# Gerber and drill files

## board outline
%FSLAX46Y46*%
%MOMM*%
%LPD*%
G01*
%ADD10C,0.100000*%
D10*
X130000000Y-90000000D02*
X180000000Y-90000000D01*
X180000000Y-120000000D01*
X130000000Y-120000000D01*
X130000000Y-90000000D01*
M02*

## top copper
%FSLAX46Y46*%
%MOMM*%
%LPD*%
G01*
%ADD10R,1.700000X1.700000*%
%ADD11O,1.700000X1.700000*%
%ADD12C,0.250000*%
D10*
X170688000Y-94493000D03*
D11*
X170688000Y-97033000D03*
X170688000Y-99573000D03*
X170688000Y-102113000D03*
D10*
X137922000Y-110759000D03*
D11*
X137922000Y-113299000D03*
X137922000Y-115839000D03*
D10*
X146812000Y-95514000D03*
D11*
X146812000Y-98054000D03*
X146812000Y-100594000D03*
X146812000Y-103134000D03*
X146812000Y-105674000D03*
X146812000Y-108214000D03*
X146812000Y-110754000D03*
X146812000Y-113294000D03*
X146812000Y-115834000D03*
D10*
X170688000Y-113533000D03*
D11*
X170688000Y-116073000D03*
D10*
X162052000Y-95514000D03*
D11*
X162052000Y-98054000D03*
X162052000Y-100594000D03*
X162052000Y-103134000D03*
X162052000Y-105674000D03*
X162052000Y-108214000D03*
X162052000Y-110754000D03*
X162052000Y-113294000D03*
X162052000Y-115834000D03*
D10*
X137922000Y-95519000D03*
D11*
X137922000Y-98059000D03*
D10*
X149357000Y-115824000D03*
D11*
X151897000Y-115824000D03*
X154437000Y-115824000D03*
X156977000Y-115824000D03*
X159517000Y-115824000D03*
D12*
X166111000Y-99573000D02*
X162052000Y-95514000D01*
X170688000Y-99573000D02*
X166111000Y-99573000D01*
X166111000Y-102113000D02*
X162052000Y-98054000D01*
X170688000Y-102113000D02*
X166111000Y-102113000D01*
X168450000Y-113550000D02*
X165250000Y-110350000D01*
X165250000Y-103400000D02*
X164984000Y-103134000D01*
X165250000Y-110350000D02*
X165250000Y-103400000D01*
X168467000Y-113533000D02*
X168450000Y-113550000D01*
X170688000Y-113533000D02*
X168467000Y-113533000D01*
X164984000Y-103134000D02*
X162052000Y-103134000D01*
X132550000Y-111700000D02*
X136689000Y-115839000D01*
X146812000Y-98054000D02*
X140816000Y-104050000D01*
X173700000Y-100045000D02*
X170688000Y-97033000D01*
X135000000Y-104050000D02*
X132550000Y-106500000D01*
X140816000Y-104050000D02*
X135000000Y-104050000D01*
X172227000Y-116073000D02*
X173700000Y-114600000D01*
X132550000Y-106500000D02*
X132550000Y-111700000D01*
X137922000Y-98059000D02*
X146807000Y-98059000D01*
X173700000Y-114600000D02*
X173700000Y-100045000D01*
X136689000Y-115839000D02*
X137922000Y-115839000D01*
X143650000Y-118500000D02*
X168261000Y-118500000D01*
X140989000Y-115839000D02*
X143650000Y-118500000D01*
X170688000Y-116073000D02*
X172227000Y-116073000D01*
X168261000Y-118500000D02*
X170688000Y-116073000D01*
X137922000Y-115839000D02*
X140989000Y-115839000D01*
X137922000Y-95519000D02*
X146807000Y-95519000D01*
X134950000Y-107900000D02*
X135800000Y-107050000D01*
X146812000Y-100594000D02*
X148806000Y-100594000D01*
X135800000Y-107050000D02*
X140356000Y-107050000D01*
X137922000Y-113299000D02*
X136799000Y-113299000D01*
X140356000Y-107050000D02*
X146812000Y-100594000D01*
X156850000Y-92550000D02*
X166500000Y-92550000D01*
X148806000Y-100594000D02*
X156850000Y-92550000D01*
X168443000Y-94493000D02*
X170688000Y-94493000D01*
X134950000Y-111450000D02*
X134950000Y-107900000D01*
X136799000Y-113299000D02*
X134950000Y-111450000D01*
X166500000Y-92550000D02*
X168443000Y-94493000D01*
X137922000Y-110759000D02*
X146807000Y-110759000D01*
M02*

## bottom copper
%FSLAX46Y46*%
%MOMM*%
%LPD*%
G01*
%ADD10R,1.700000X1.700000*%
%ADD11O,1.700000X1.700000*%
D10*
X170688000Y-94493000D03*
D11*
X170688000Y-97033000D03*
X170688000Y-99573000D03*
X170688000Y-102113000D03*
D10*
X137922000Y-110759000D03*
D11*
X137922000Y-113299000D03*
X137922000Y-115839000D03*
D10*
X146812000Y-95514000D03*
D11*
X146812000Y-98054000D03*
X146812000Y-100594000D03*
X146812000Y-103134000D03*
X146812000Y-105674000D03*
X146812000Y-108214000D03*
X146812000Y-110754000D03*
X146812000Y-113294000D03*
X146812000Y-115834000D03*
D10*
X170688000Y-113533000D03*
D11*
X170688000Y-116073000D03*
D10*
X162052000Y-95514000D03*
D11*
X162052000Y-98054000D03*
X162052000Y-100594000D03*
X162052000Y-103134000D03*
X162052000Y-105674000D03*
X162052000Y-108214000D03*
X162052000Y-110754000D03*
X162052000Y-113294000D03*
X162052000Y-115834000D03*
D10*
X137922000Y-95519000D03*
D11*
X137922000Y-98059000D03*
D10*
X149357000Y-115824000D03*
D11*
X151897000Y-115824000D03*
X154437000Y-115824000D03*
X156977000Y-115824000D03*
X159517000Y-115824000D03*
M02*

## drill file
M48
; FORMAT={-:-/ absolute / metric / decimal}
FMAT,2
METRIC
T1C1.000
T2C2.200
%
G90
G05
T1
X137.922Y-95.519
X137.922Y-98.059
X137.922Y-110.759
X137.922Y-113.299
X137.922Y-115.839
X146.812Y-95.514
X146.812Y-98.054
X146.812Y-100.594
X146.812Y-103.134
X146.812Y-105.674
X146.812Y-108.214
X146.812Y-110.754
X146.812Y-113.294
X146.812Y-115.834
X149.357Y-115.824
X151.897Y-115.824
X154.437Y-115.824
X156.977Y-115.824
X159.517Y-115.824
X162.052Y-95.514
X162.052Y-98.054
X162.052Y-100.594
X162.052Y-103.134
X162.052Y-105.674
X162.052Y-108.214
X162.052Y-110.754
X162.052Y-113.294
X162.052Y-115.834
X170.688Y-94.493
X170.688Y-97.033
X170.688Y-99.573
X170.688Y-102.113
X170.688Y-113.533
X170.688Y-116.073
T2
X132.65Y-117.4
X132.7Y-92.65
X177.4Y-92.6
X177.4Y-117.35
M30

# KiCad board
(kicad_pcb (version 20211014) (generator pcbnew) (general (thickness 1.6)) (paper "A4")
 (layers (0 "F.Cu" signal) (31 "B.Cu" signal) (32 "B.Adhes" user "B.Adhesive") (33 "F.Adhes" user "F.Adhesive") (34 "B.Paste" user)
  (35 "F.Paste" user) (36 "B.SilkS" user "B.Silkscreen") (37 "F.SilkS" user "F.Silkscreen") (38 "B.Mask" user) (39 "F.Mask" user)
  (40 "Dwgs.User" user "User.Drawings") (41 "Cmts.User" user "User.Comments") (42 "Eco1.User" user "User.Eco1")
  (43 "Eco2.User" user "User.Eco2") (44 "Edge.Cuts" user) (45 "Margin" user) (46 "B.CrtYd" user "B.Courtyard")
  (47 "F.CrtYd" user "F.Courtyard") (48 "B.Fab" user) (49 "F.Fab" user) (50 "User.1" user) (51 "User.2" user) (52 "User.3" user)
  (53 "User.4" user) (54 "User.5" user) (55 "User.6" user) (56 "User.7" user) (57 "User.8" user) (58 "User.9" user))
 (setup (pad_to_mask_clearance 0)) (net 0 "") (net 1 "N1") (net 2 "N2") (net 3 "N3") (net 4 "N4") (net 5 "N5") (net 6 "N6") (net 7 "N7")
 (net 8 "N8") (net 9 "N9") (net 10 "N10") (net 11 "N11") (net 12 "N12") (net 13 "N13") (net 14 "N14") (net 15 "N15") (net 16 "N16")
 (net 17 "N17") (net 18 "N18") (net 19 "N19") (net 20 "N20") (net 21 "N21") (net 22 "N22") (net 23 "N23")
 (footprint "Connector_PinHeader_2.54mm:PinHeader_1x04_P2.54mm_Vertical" (layer "F.Cu") (at 170.688 94.493)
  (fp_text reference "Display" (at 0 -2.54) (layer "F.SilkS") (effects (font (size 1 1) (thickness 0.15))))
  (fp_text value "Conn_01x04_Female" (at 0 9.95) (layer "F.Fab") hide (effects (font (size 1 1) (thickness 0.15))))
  (pad "1" thru_hole rect (at 0 0) (size 1.7 1.7) (drill 1) (layers *.Cu *.Mask) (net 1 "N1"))
  (pad "2" thru_hole oval (at 0 2.54) (size 1.7 1.7) (drill 1) (layers *.Cu *.Mask) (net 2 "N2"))
  (pad "3" thru_hole oval (at 0 5.08) (size 1.7 1.7) (drill 1) (layers *.Cu *.Mask) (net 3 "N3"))
  (pad "4" thru_hole oval (at 0 7.62) (size 1.7 1.7) (drill 1) (layers *.Cu *.Mask) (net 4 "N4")))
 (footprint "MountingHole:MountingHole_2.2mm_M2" (layer "F.Cu") (at 177.4 92.6)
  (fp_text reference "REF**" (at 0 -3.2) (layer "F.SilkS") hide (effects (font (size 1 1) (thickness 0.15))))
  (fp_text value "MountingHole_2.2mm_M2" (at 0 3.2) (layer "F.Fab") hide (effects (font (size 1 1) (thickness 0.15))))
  (pad "" np_thru_hole circle (at 0 0) (size 2.2 2.2) (drill 2.2) (layers *.Cu *.Mask)))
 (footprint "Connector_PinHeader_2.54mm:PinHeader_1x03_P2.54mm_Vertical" (layer "F.Cu") (at 137.922 110.759)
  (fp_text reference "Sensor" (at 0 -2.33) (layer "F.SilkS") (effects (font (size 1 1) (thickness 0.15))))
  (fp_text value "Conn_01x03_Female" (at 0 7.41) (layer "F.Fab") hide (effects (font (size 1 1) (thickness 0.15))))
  (pad "1" thru_hole rect (at 0 0) (size 1.7 1.7) (drill 1) (layers *.Cu *.Mask) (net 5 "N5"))
  (pad "2" thru_hole oval (at 0 2.54) (size 1.7 1.7) (drill 1) (layers *.Cu *.Mask) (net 1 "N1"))
  (pad "3" thru_hole oval (at 0 5.08) (size 1.7 1.7) (drill 1) (layers *.Cu *.Mask) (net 2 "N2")))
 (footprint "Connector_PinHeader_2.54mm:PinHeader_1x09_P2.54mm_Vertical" (layer "F.Cu") (at 146.812 95.514)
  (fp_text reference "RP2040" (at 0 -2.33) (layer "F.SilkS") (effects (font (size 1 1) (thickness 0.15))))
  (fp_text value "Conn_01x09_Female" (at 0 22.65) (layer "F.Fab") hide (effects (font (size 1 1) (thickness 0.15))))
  (pad "1" thru_hole rect (at 0 0) (size 1.7 1.7) (drill 1) (layers *.Cu *.Mask) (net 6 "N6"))
  (pad "2" thru_hole oval (at 0 2.54) (size 1.7 1.7) (drill 1) (layers *.Cu *.Mask) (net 2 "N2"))
  (pad "3" thru_hole oval (at 0 5.08) (size 1.7 1.7) (drill 1) (layers *.Cu *.Mask) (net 1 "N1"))
  (pad "4" thru_hole oval (at 0 7.62) (size 1.7 1.7) (drill 1) (layers *.Cu *.Mask) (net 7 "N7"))
  (pad "5" thru_hole oval (at 0 10.16) (size 1.7 1.7) (drill 1) (layers *.Cu *.Mask) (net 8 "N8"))
  (pad "6" thru_hole oval (at 0 12.7) (size 1.7 1.7) (drill 1) (layers *.Cu *.Mask) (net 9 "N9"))
  (pad "7" thru_hole oval (at 0 15.24) (size 1.7 1.7) (drill 1) (layers *.Cu *.Mask) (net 5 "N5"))
  (pad "8" thru_hole oval (at 0 17.78) (size 1.7 1.7) (drill 1) (layers *.Cu *.Mask) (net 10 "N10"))
  (pad "9" thru_hole oval (at 0 20.32) (size 1.7 1.7) (drill 1) (layers *.Cu *.Mask) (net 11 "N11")))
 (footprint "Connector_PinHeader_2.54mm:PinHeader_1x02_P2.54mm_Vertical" (layer "F.Cu") (at 170.688 113.533)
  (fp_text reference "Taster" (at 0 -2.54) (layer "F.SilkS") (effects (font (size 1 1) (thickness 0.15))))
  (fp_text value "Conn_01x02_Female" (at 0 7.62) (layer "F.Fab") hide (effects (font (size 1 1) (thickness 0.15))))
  (pad "1" thru_hole rect (at 0 0) (size 1.7 1.7) (drill 1) (layers *.Cu *.Mask) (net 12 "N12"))
  (pad "2" thru_hole oval (at 0 2.54) (size 1.7 1.7) (drill 1) (layers *.Cu *.Mask) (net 2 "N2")))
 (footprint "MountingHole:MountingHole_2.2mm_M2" (layer "F.Cu") (at 132.7 92.65)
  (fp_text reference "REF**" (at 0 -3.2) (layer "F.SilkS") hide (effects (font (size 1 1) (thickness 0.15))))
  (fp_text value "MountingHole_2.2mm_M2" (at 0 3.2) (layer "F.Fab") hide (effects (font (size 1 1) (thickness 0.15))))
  (pad "" np_thru_hole circle (at 0 0) (size 2.2 2.2) (drill 2.2) (layers *.Cu *.Mask)))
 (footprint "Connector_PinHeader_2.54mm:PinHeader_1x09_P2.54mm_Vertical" (layer "F.Cu") (at 162.052 95.514)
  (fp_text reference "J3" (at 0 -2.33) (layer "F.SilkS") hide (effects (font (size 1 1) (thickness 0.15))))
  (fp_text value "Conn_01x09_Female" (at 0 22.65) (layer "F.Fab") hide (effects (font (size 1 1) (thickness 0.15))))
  (pad "1" thru_hole rect (at 0 0) (size 1.7 1.7) (drill 1) (layers *.Cu *.Mask) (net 3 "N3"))
  (pad "2" thru_hole oval (at 0 2.54) (size 1.7 1.7) (drill 1) (layers *.Cu *.Mask) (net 4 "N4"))
  (pad "3" thru_hole oval (at 0 5.08) (size 1.7 1.7) (drill 1) (layers *.Cu *.Mask) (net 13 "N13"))
  (pad "4" thru_hole oval (at 0 7.62) (size 1.7 1.7) (drill 1) (layers *.Cu *.Mask) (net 12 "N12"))
  (pad "5" thru_hole oval (at 0 10.16) (size 1.7 1.7) (drill 1) (layers *.Cu *.Mask) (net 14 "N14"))
  (pad "6" thru_hole oval (at 0 12.7) (size 1.7 1.7) (drill 1) (layers *.Cu *.Mask) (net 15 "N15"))
  (pad "7" thru_hole oval (at 0 15.24) (size 1.7 1.7) (drill 1) (layers *.Cu *.Mask) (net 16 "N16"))
  (pad "8" thru_hole oval (at 0 17.78) (size 1.7 1.7) (drill 1) (layers *.Cu *.Mask) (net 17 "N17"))
  (pad "9" thru_hole oval (at 0 20.32) (size 1.7 1.7) (drill 1) (layers *.Cu *.Mask) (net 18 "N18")))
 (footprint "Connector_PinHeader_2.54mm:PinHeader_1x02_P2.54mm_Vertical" (layer "F.Cu") (at 137.922 95.519)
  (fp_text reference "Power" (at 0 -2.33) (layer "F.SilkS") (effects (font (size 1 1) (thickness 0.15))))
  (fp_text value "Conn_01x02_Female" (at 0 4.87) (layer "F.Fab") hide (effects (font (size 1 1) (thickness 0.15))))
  (pad "1" thru_hole rect (at 0 0) (size 1.7 1.7) (drill 1) (layers *.Cu *.Mask) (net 6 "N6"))
  (pad "2" thru_hole oval (at 0 2.54) (size 1.7 1.7) (drill 1) (layers *.Cu *.Mask) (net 2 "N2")))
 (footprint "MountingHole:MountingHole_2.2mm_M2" (layer "F.Cu") (at 177.4 117.35)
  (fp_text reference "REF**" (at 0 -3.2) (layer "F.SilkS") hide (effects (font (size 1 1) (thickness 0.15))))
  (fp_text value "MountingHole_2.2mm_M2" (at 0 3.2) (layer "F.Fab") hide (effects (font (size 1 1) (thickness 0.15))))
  (pad "" np_thru_hole circle (at 0 0) (size 2.2 2.2) (drill 2.2) (layers *.Cu *.Mask)))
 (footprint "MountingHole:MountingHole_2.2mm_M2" (layer "F.Cu") (at 132.65 117.4)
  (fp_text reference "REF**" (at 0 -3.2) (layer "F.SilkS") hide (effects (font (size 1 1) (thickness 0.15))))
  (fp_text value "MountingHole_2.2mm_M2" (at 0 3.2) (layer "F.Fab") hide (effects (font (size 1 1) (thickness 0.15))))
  (pad "" np_thru_hole circle (at 0 0) (size 2.2 2.2) (drill 2.2) (layers *.Cu *.Mask)))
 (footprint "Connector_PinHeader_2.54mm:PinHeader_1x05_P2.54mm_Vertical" (layer "F.Cu") (at 149.357 115.824 90)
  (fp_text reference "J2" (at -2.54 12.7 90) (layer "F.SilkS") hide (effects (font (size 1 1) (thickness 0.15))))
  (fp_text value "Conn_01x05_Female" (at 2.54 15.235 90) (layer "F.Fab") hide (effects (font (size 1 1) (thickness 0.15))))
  (pad "1" thru_hole rect (at 0 0 90) (size 1.7 1.7) (drill 1) (layers *.Cu *.Mask) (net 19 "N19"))
  (pad "2" thru_hole oval (at 0 2.54 90) (size 1.7 1.7) (drill 1) (layers *.Cu *.Mask) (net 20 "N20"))
  (pad "3" thru_hole oval (at 0 5.08 90) (size 1.7 1.7) (drill 1) (layers *.Cu *.Mask) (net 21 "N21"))
  (pad "4" thru_hole oval (at 0 7.62 90) (size 1.7 1.7) (drill 1) (layers *.Cu *.Mask) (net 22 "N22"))
  (pad "5" thru_hole oval (at 0 10.16 90) (size 1.7 1.7) (drill 1) (layers *.Cu *.Mask) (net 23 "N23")))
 (gr_rect (start 130 90) (end 180 120) (layer "Edge.Cuts") (width 0.1) (fill none))
 (gr_rect (start 99.06 43.18) (end 99.06 43.18) (layer "Edge.Cuts") (width 0.1) (fill none))
 (segment (start 166.111 99.573) (end 162.052 95.514) (width 0.25) (layer "F.Cu") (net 3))
 (segment (start 170.688 99.573) (end 166.111 99.573) (width 0.25) (layer "F.Cu") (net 3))
 (segment (start 166.111 102.113) (end 162.052 98.054) (width 0.25) (layer "F.Cu") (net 4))
 (segment (start 170.688 102.113) (end 166.111 102.113) (width 0.25) (layer "F.Cu") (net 4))
 (segment (start 168.45 113.55) (end 165.25 110.35) (width 0.25) (layer "F.Cu") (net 12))
 (segment (start 165.25 103.4) (end 164.984 103.134) (width 0.25) (layer "F.Cu") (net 12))
 (segment (start 165.25 110.35) (end 165.25 103.4) (width 0.25) (layer "F.Cu") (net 12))
 (segment (start 168.467 113.533) (end 168.45 113.55) (width 0.25) (layer "F.Cu") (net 12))
 (segment (start 170.688 113.533) (end 168.467 113.533) (width 0.25) (layer "F.Cu") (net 12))
 (segment (start 164.984 103.134) (end 162.052 103.134) (width 0.25) (layer "F.Cu") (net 12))
 (segment (start 132.55 111.7) (end 136.689 115.839) (width 0.25) (layer "F.Cu") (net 2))
 (segment (start 146.812 98.054) (end 140.816 104.05) (width 0.25) (layer "F.Cu") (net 2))
 (segment (start 173.7 100.045) (end 170.688 97.033) (width 0.25) (layer "F.Cu") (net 2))
 (segment (start 135 104.05) (end 132.55 106.5) (width 0.25) (layer "F.Cu") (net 2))
 (segment (start 140.816 104.05) (end 135 104.05) (width 0.25) (layer "F.Cu") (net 2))
 (segment (start 172.227 116.073) (end 173.7 114.6) (width 0.25) (layer "F.Cu") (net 2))
 (segment (start 132.55 106.5) (end 132.55 111.7) (width 0.25) (layer "F.Cu") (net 2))
 (segment (start 137.922 98.059) (end 146.807 98.059) (width 0.25) (layer "F.Cu") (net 2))
 (segment (start 173.7 114.6) (end 173.7 100.045) (width 0.25) (layer "F.Cu") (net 2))
 (segment (start 136.689 115.839) (end 137.922 115.839) (width 0.25) (layer "F.Cu") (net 2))
 (segment (start 143.65 118.5) (end 168.261 118.5) (width 0.25) (layer "F.Cu") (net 2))
 (segment (start 140.989 115.839) (end 143.65 118.5) (width 0.25) (layer "F.Cu") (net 2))
 (segment (start 170.688 116.073) (end 172.227 116.073) (width 0.25) (layer "F.Cu") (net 2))
 (segment (start 168.261 118.5) (end 170.688 116.073) (width 0.25) (layer "F.Cu") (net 2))
 (segment (start 137.922 115.839) (end 140.989 115.839) (width 0.25) (layer "F.Cu") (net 2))
 (segment (start 137.922 95.519) (end 146.807 95.519) (width 0.25) (layer "F.Cu") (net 6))
 (segment (start 134.95 107.9) (end 135.8 107.05) (width 0.25) (layer "F.Cu") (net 1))
 (segment (start 146.812 100.594) (end 148.806 100.594) (width 0.25) (layer "F.Cu") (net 1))
 (segment (start 135.8 107.05) (end 140.356 107.05) (width 0.25) (layer "F.Cu") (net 1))
 (segment (start 137.922 113.299) (end 136.799 113.299) (width 0.25) (layer "F.Cu") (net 1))
 (segment (start 140.356 107.05) (end 146.812 100.594) (width 0.25) (layer "F.Cu") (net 1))
 (segment (start 156.85 92.55) (end 166.5 92.55) (width 0.25) (layer "F.Cu") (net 1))
 (segment (start 148.806 100.594) (end 156.85 92.55) (width 0.25) (layer "F.Cu") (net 1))
 (segment (start 168.443 94.493) (end 170.688 94.493) (width 0.25) (layer "F.Cu") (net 1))
 (segment (start 134.95 111.45) (end 134.95 107.9) (width 0.25) (layer "F.Cu") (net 1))
 (segment (start 136.799 113.299) (end 134.95 111.45) (width 0.25) (layer "F.Cu") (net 1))
 (segment (start 166.5 92.55) (end 168.443 94.493) (width 0.25) (layer "F.Cu") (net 1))
 (segment (start 137.922 110.759) (end 146.807 110.759) (width 0.25) (layer "F.Cu") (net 5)))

